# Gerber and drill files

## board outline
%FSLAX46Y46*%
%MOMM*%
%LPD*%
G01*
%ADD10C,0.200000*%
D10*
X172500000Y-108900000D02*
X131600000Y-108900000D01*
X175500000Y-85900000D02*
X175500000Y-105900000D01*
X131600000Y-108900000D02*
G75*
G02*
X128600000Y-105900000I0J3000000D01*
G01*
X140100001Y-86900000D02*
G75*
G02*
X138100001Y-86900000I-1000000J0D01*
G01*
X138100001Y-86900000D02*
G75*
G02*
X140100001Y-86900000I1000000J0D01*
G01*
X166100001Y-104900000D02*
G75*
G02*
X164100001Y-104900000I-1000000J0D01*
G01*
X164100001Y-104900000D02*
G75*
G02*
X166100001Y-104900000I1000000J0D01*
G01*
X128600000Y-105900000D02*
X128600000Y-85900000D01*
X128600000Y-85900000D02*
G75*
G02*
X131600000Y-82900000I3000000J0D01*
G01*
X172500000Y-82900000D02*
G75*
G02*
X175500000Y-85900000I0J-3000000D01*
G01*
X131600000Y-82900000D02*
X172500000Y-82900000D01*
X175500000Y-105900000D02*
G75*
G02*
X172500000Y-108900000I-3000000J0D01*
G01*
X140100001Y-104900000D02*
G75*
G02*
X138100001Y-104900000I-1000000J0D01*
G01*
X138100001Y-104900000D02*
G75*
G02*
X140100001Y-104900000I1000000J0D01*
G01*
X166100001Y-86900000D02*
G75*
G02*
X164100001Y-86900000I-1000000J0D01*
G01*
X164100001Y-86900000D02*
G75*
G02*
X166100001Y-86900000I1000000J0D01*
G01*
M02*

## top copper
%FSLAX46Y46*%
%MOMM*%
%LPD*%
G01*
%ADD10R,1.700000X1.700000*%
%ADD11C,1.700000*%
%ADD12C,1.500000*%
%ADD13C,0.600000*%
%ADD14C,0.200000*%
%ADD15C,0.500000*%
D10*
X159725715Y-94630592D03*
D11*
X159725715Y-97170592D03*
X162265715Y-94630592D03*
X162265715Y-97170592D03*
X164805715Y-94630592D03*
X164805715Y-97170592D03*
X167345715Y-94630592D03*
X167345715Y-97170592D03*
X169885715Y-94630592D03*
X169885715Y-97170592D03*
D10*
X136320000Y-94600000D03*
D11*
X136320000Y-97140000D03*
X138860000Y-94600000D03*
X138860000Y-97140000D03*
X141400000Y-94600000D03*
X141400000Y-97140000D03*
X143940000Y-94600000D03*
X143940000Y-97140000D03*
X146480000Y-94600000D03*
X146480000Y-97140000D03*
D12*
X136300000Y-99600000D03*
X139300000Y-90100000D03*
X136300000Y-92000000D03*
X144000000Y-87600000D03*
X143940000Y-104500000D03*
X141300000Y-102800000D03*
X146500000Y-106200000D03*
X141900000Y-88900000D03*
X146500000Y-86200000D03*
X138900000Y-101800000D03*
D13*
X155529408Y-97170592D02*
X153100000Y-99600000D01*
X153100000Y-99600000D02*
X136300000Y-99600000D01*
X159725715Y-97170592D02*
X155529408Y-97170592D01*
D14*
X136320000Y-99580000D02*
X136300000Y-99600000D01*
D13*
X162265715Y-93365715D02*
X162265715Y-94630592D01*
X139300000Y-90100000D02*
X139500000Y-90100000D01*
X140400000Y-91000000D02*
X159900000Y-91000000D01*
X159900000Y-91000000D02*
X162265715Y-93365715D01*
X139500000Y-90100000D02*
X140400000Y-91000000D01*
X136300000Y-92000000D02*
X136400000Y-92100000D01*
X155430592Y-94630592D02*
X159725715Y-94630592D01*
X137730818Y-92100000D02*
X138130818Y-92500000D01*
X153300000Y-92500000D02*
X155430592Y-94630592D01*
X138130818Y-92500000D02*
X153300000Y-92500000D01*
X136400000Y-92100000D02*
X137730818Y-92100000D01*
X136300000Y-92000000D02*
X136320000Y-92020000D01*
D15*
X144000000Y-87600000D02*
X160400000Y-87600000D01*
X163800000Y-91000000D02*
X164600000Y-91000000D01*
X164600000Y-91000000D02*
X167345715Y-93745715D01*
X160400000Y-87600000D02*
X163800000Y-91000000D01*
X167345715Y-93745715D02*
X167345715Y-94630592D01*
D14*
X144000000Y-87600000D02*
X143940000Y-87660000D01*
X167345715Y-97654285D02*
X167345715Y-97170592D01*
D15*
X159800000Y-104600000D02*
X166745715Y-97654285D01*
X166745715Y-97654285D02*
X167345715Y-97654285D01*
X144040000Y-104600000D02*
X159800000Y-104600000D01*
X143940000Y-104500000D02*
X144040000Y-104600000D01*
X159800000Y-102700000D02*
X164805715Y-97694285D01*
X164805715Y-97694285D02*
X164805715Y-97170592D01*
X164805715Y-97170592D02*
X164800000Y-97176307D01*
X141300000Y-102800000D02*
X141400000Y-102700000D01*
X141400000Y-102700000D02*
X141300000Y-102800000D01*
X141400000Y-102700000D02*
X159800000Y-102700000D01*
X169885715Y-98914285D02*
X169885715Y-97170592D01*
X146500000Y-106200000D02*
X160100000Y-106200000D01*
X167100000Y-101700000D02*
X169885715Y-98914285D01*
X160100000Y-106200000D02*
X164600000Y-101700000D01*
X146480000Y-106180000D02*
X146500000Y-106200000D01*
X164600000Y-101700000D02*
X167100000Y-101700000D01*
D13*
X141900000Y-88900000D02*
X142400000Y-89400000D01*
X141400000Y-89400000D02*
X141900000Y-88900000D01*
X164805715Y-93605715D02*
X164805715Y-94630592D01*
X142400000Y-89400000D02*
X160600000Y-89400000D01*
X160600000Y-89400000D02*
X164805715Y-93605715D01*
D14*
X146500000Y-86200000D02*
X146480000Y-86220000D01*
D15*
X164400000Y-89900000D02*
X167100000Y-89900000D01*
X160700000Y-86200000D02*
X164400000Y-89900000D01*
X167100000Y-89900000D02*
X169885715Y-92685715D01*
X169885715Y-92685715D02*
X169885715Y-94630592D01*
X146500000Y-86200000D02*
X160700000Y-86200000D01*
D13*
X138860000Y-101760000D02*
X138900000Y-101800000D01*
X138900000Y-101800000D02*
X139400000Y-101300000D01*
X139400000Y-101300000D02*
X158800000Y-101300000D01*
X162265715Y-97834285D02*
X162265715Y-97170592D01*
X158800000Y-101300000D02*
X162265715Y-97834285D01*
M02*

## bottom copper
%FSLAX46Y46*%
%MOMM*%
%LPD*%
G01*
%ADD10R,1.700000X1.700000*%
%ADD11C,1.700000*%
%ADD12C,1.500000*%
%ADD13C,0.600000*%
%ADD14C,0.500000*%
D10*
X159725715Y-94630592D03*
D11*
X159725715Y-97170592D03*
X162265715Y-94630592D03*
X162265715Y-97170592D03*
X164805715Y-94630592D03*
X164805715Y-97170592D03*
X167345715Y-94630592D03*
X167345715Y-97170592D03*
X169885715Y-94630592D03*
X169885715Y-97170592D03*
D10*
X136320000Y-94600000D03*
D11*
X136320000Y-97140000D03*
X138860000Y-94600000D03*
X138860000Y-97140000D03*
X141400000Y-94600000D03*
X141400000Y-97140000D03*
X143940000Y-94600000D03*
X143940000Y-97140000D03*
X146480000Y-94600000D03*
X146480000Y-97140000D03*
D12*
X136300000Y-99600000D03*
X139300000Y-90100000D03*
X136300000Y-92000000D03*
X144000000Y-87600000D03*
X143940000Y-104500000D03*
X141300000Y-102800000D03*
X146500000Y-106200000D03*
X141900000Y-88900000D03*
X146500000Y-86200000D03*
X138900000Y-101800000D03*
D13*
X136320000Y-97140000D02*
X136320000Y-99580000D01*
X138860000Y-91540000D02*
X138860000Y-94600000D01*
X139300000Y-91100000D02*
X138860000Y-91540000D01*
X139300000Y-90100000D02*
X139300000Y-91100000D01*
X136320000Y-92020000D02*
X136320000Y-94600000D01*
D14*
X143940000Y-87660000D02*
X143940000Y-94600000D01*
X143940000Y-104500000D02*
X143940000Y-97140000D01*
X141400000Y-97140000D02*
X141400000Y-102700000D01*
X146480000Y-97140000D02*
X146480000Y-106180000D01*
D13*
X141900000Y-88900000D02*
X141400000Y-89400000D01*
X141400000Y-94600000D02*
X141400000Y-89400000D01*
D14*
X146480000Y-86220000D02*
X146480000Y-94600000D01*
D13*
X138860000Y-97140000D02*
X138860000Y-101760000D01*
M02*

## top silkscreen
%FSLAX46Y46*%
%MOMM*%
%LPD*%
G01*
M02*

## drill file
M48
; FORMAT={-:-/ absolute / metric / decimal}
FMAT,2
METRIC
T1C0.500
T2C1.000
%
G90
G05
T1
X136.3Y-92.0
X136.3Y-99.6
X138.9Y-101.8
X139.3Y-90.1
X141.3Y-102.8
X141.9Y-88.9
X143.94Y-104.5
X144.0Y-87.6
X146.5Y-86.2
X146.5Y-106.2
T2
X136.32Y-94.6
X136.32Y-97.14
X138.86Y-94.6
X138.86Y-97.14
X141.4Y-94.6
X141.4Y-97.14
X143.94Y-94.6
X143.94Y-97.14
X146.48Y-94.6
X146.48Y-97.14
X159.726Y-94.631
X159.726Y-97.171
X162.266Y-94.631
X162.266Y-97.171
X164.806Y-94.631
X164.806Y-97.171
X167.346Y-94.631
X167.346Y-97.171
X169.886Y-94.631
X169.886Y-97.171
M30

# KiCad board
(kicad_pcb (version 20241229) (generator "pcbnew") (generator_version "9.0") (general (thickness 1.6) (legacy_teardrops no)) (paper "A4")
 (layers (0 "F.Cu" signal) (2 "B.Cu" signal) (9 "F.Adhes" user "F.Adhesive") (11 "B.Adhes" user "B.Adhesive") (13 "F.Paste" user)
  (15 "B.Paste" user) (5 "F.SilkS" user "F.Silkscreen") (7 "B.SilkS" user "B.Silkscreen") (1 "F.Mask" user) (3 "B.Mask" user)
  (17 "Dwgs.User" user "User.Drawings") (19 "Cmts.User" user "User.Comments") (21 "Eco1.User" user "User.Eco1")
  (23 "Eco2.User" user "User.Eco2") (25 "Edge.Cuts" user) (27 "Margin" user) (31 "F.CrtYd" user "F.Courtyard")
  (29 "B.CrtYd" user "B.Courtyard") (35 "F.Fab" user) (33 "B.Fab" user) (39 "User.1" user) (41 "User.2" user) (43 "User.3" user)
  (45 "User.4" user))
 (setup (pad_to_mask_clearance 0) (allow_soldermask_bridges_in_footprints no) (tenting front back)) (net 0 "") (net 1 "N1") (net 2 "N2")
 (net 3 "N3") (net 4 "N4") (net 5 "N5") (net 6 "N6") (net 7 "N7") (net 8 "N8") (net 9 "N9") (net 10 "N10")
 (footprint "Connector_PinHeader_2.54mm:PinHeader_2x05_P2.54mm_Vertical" (layer "B.Cu") (at 159.725715 94.630592 -90)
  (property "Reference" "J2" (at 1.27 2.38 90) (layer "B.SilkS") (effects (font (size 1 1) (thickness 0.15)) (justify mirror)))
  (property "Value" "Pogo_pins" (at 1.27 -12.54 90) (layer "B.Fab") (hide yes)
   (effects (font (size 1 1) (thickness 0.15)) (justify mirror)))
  (pad "1" thru_hole rect (at 0 0 270) (size 1.7 1.7) (drill 1) (layers "*.Cu" "*.Mask") (remove_unused_layers no) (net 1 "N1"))
  (pad "2" thru_hole circle (at 2.54 0 270) (size 1.7 1.7) (drill 1) (layers "*.Cu" "*.Mask") (remove_unused_layers no) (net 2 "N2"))
  (pad "3" thru_hole circle (at 0 -2.54 270) (size 1.7 1.7) (drill 1) (layers "*.Cu" "*.Mask") (remove_unused_layers no) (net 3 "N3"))
  (pad "4" thru_hole circle (at 2.54 -2.54 270) (size 1.7 1.7) (drill 1) (layers "*.Cu" "*.Mask") (remove_unused_layers no) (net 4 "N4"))
  (pad "5" thru_hole circle (at 0 -5.08 270) (size 1.7 1.7) (drill 1) (layers "*.Cu" "*.Mask") (remove_unused_layers no) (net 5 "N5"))
  (pad "6" thru_hole circle (at 2.54 -5.08 270) (size 1.7 1.7) (drill 1) (layers "*.Cu" "*.Mask") (remove_unused_layers no) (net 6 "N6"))
  (pad "7" thru_hole circle (at 0 -7.62 270) (size 1.7 1.7) (drill 1) (layers "*.Cu" "*.Mask") (remove_unused_layers no) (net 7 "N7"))
  (pad "8" thru_hole circle (at 2.54 -7.62 270) (size 1.7 1.7) (drill 1) (layers "*.Cu" "*.Mask") (remove_unused_layers no) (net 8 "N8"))
  (pad "9" thru_hole circle (at 0 -10.16 270) (size 1.7 1.7) (drill 1) (layers "*.Cu" "*.Mask") (remove_unused_layers no) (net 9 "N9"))
  (pad "10" thru_hole circle (at 2.54 -10.16 270) (size 1.7 1.7) (drill 1) (layers "*.Cu" "*.Mask") (remove_unused_layers no) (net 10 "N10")))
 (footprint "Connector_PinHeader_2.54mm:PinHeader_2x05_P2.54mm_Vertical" (layer "B.Cu") (at 136.32 94.6 -90)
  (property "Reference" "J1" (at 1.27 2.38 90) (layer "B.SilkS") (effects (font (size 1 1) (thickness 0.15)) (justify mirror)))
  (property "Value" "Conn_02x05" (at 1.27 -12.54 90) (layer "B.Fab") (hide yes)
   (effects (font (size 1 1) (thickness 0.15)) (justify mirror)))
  (pad "1" thru_hole rect (at 0 0 270) (size 1.7 1.7) (drill 1) (layers "*.Cu" "*.Mask") (remove_unused_layers no) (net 1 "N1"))
  (pad "2" thru_hole circle (at 2.54 0 270) (size 1.7 1.7) (drill 1) (layers "*.Cu" "*.Mask") (remove_unused_layers no) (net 2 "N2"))
  (pad "3" thru_hole circle (at 0 -2.54 270) (size 1.7 1.7) (drill 1) (layers "*.Cu" "*.Mask") (remove_unused_layers no) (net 3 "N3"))
  (pad "4" thru_hole circle (at 2.54 -2.54 270) (size 1.7 1.7) (drill 1) (layers "*.Cu" "*.Mask") (remove_unused_layers no) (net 4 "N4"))
  (pad "5" thru_hole circle (at 0 -5.08 270) (size 1.7 1.7) (drill 1) (layers "*.Cu" "*.Mask") (remove_unused_layers no) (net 5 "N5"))
  (pad "6" thru_hole circle (at 2.54 -5.08 270) (size 1.7 1.7) (drill 1) (layers "*.Cu" "*.Mask") (remove_unused_layers no) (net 6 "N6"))
  (pad "7" thru_hole circle (at 0 -7.62 270) (size 1.7 1.7) (drill 1) (layers "*.Cu" "*.Mask") (remove_unused_layers no) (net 7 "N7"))
  (pad "8" thru_hole circle (at 2.54 -7.62 270) (size 1.7 1.7) (drill 1) (layers "*.Cu" "*.Mask") (remove_unused_layers no) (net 8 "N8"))
  (pad "9" thru_hole circle (at 0 -10.16 270) (size 1.7 1.7) (drill 1) (layers "*.Cu" "*.Mask") (remove_unused_layers no) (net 9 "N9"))
  (pad "10" thru_hole circle (at 2.54 -10.16 270) (size 1.7 1.7) (drill 1) (layers "*.Cu" "*.Mask") (remove_unused_layers no) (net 10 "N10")))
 (gr_line (start 172.5 108.9) (end 131.6 108.9) (stroke (width 0.2) (type default)) (layer "Edge.Cuts"))
 (gr_line (start 175.5 85.9) (end 175.5 105.9) (stroke (width 0.2) (type default)) (layer "Edge.Cuts"))
 (gr_arc (start 131.6 108.9) (mid 129.47868 108.02132) (end 128.6 105.9) (stroke (width 0.2) (type default)) (layer "Edge.Cuts"))
 (gr_circle (center 139.100001 86.9) (end 140.100001 86.9) (stroke (width 0.2) (type solid)) (fill no) (layer "Edge.Cuts"))
 (gr_circle (center 165.100001 104.9) (end 166.100001 104.9) (stroke (width 0.2) (type solid)) (fill no) (layer "Edge.Cuts"))
 (gr_line (start 128.6 105.9) (end 128.6 85.9) (stroke (width 0.2) (type default)) (layer "Edge.Cuts"))
 (gr_arc (start 128.6 85.9) (mid 129.47868 83.77868) (end 131.6 82.9) (stroke (width 0.2) (type default)) (layer "Edge.Cuts"))
 (gr_arc (start 172.5 82.9) (mid 174.62132 83.77868) (end 175.5 85.9) (stroke (width 0.2) (type default)) (layer "Edge.Cuts"))
 (gr_line (start 131.6 82.9) (end 172.5 82.9) (stroke (width 0.2) (type default)) (layer "Edge.Cuts"))
 (gr_arc (start 175.5 105.9) (mid 174.62132 108.02132) (end 172.5 108.9) (stroke (width 0.2) (type default)) (layer "Edge.Cuts"))
 (gr_circle (center 139.100001 104.9) (end 140.100001 104.9) (stroke (width 0.2) (type solid)) (fill no) (layer "Edge.Cuts"))
 (gr_circle (center 165.100001 86.9) (end 166.100001 86.9) (stroke (width 0.2) (type solid)) (fill no) (layer "Edge.Cuts"))
 (segment (start 155.529408 97.170592) (end 153.1 99.6) (width 0.6) (layer "F.Cu") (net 2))
 (segment (start 153.1 99.6) (end 136.3 99.6) (width 0.6) (layer "F.Cu") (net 2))
 (segment (start 159.725715 97.170592) (end 155.529408 97.170592) (width 0.6) (layer "F.Cu") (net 2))
 (segment (start 136.32 99.58) (end 136.3 99.6) (width 0.2) (layer "F.Cu") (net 2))
 (via (at 136.3 99.6) (size 1.5) (drill 0.5) (layers "F.Cu" "B.Cu") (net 2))
 (segment (start 136.32 97.14) (end 136.32 99.58) (width 0.6) (layer "B.Cu") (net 2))
 (segment (start 162.265715 93.365715) (end 162.265715 94.630592) (width 0.6) (layer "F.Cu") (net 3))
 (segment (start 139.3 90.1) (end 139.5 90.1) (width 0.6) (layer "F.Cu") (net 3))
 (segment (start 140.4 91) (end 159.9 91) (width 0.6) (layer "F.Cu") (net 3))
 (segment (start 159.9 91) (end 162.265715 93.365715) (width 0.6) (layer "F.Cu") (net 3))
 (segment (start 139.5 90.1) (end 140.4 91) (width 0.6) (layer "F.Cu") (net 3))
 (via (at 139.3 90.1) (size 1.5) (drill 0.5) (layers "F.Cu" "B.Cu") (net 3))
 (segment (start 138.86 91.54) (end 138.86 94.6) (width 0.6) (layer "B.Cu") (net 3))
 (segment (start 139.3 91.1) (end 138.86 91.54) (width 0.6) (layer "B.Cu") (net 3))
 (segment (start 139.3 90.1) (end 139.3 91.1) (width 0.6) (layer "B.Cu") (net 3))
 (segment (start 136.3 92) (end 136.4 92.1) (width 0.6) (layer "F.Cu") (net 1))
 (segment (start 155.430592 94.630592) (end 159.725715 94.630592) (width 0.6) (layer "F.Cu") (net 1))
 (segment (start 137.730818 92.1) (end 138.130818 92.5) (width 0.6) (layer "F.Cu") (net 1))
 (segment (start 153.3 92.5) (end 155.430592 94.630592) (width 0.6) (layer "F.Cu") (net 1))
 (segment (start 138.130818 92.5) (end 153.3 92.5) (width 0.6) (layer "F.Cu") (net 1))
 (segment (start 136.4 92.1) (end 137.730818 92.1) (width 0.6) (layer "F.Cu") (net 1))
 (segment (start 136.3 92) (end 136.32 92.02) (width 0.6) (layer "F.Cu") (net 1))
 (via (at 136.3 92) (size 1.5) (drill 0.5) (layers "F.Cu" "B.Cu") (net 1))
 (segment (start 136.32 92.02) (end 136.32 94.6) (width 0.6) (layer "B.Cu") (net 1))
 (segment (start 144 87.6) (end 160.4 87.6) (width 0.5) (layer "F.Cu") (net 7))
 (segment (start 163.8 91) (end 164.6 91) (width 0.5) (layer "F.Cu") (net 7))
 (segment (start 164.6 91) (end 167.345715 93.745715) (width 0.5) (layer "F.Cu") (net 7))
 (segment (start 160.4 87.6) (end 163.8 91) (width 0.5) (layer "F.Cu") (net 7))
 (segment (start 167.345715 93.745715) (end 167.345715 94.630592) (width 0.5) (layer "F.Cu") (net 7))
 (segment (start 144 87.6) (end 143.94 87.66) (width 0.2) (layer "F.Cu") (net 7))
 (via (at 144 87.6) (size 1.5) (drill 0.5) (layers "F.Cu" "B.Cu") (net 7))
 (segment (start 143.94 87.66) (end 143.94 94.6) (width 0.5) (layer "B.Cu") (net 7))
 (segment (start 167.345715 97.654285) (end 167.345715 97.170592) (width 0.2) (layer "F.Cu") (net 8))
 (segment (start 159.8 104.6) (end 166.745715 97.654285) (width 0.5) (layer "F.Cu") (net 8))
 (segment (start 166.745715 97.654285) (end 167.345715 97.654285) (width 0.5) (layer "F.Cu") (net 8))
 (segment (start 144.04 104.6) (end 159.8 104.6) (width 0.5) (layer "F.Cu") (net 8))
 (segment (start 143.94 104.5) (end 144.04 104.6) (width 0.5) (layer "F.Cu") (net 8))
 (via (at 143.94 104.5) (size 1.5) (drill 0.5) (layers "F.Cu" "B.Cu") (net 8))
 (segment (start 143.94 104.5) (end 143.94 97.14) (width 0.5) (layer "B.Cu") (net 8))
 (segment (start 159.8 102.7) (end 164.805715 97.694285) (width 0.5) (layer "F.Cu") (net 6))
 (segment (start 164.805715 97.694285) (end 164.805715 97.170592) (width 0.5) (layer "F.Cu") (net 6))
 (segment (start 164.805715 97.170592) (end 164.8 97.176307) (width 0.5) (layer "F.Cu") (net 6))
 (segment (start 141.3 102.8) (end 141.4 102.7) (width 0.5) (layer "F.Cu") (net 6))
 (segment (start 141.4 102.7) (end 141.3 102.8) (width 0.5) (layer "F.Cu") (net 6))
 (segment (start 141.4 102.7) (end 159.8 102.7) (width 0.5) (layer "F.Cu") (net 6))
 (via (at 141.3 102.8) (size 1.5) (drill 0.5) (layers "F.Cu" "B.Cu") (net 6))
 (segment (start 141.4 97.14) (end 141.4 102.7) (width 0.5) (layer "B.Cu") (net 6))
 (segment (start 169.885715 98.914285) (end 169.885715 97.170592) (width 0.5) (layer "F.Cu") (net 10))
 (segment (start 146.5 106.2) (end 160.1 106.2) (width 0.5) (layer "F.Cu") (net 10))
 (segment (start 167.1 101.7) (end 169.885715 98.914285) (width 0.5) (layer "F.Cu") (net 10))
 (segment (start 160.1 106.2) (end 164.6 101.7) (width 0.5) (layer "F.Cu") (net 10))
 (segment (start 146.48 106.18) (end 146.5 106.2) (width 0.5) (layer "F.Cu") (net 10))
 (segment (start 164.6 101.7) (end 167.1 101.7) (width 0.5) (layer "F.Cu") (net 10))
 (via (at 146.5 106.2) (size 1.5) (drill 0.5) (layers "F.Cu" "B.Cu") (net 10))
 (segment (start 146.48 97.14) (end 146.48 106.18) (width 0.5) (layer "B.Cu") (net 10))
 (segment (start 141.9 88.9) (end 142.4 89.4) (width 0.6) (layer "F.Cu") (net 5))
 (segment (start 141.4 89.4) (end 141.9 88.9) (width 0.6) (layer "F.Cu") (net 5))
 (segment (start 164.805715 93.605715) (end 164.805715 94.630592) (width 0.6) (layer "F.Cu") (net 5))
 (segment (start 142.4 89.4) (end 160.6 89.4) (width 0.6) (layer "F.Cu") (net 5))
 (segment (start 160.6 89.4) (end 164.805715 93.605715) (width 0.6) (layer "F.Cu") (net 5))
 (via (at 141.9 88.9) (size 1.5) (drill 0.5) (layers "F.Cu" "B.Cu") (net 5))
 (segment (start 141.9 88.9) (end 141.4 89.4) (width 0.6) (layer "B.Cu") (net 5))
 (segment (start 141.4 94.6) (end 141.4 89.4) (width 0.6) (layer "B.Cu") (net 5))
 (segment (start 146.5 86.2) (end 146.48 86.22) (width 0.2) (layer "F.Cu") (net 9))
 (segment (start 164.4 89.9) (end 167.1 89.9) (width 0.5) (layer "F.Cu") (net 9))
 (segment (start 160.7 86.2) (end 164.4 89.9) (width 0.5) (layer "F.Cu") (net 9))
 (segment (start 167.1 89.9) (end 169.885715 92.685715) (width 0.5) (layer "F.Cu") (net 9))
 (segment (start 169.885715 92.685715) (end 169.885715 94.630592) (width 0.5) (layer "F.Cu") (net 9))
 (segment (start 146.5 86.2) (end 160.7 86.2) (width 0.5) (layer "F.Cu") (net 9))
 (via (at 146.5 86.2) (size 1.5) (drill 0.5) (layers "F.Cu" "B.Cu") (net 9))
 (segment (start 146.48 86.22) (end 146.48 94.6) (width 0.5) (layer "B.Cu") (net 9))
 (segment (start 138.86 101.76) (end 138.9 101.8) (width 0.6) (layer "F.Cu") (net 4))
 (segment (start 138.9 101.8) (end 139.4 101.3) (width 0.6) (layer "F.Cu") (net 4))
 (segment (start 139.4 101.3) (end 158.8 101.3) (width 0.6) (layer "F.Cu") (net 4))
 (segment (start 162.265715 97.834285) (end 162.265715 97.170592) (width 0.6) (layer "F.Cu") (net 4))
 (segment (start 158.8 101.3) (end 162.265715 97.834285) (width 0.6) (layer "F.Cu") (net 4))
 (via (at 138.9 101.8) (size 1.5) (drill 0.5) (layers "F.Cu" "B.Cu") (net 4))
 (segment (start 138.86 97.14) (end 138.86 101.76) (width 0.6) (layer "B.Cu") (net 4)))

